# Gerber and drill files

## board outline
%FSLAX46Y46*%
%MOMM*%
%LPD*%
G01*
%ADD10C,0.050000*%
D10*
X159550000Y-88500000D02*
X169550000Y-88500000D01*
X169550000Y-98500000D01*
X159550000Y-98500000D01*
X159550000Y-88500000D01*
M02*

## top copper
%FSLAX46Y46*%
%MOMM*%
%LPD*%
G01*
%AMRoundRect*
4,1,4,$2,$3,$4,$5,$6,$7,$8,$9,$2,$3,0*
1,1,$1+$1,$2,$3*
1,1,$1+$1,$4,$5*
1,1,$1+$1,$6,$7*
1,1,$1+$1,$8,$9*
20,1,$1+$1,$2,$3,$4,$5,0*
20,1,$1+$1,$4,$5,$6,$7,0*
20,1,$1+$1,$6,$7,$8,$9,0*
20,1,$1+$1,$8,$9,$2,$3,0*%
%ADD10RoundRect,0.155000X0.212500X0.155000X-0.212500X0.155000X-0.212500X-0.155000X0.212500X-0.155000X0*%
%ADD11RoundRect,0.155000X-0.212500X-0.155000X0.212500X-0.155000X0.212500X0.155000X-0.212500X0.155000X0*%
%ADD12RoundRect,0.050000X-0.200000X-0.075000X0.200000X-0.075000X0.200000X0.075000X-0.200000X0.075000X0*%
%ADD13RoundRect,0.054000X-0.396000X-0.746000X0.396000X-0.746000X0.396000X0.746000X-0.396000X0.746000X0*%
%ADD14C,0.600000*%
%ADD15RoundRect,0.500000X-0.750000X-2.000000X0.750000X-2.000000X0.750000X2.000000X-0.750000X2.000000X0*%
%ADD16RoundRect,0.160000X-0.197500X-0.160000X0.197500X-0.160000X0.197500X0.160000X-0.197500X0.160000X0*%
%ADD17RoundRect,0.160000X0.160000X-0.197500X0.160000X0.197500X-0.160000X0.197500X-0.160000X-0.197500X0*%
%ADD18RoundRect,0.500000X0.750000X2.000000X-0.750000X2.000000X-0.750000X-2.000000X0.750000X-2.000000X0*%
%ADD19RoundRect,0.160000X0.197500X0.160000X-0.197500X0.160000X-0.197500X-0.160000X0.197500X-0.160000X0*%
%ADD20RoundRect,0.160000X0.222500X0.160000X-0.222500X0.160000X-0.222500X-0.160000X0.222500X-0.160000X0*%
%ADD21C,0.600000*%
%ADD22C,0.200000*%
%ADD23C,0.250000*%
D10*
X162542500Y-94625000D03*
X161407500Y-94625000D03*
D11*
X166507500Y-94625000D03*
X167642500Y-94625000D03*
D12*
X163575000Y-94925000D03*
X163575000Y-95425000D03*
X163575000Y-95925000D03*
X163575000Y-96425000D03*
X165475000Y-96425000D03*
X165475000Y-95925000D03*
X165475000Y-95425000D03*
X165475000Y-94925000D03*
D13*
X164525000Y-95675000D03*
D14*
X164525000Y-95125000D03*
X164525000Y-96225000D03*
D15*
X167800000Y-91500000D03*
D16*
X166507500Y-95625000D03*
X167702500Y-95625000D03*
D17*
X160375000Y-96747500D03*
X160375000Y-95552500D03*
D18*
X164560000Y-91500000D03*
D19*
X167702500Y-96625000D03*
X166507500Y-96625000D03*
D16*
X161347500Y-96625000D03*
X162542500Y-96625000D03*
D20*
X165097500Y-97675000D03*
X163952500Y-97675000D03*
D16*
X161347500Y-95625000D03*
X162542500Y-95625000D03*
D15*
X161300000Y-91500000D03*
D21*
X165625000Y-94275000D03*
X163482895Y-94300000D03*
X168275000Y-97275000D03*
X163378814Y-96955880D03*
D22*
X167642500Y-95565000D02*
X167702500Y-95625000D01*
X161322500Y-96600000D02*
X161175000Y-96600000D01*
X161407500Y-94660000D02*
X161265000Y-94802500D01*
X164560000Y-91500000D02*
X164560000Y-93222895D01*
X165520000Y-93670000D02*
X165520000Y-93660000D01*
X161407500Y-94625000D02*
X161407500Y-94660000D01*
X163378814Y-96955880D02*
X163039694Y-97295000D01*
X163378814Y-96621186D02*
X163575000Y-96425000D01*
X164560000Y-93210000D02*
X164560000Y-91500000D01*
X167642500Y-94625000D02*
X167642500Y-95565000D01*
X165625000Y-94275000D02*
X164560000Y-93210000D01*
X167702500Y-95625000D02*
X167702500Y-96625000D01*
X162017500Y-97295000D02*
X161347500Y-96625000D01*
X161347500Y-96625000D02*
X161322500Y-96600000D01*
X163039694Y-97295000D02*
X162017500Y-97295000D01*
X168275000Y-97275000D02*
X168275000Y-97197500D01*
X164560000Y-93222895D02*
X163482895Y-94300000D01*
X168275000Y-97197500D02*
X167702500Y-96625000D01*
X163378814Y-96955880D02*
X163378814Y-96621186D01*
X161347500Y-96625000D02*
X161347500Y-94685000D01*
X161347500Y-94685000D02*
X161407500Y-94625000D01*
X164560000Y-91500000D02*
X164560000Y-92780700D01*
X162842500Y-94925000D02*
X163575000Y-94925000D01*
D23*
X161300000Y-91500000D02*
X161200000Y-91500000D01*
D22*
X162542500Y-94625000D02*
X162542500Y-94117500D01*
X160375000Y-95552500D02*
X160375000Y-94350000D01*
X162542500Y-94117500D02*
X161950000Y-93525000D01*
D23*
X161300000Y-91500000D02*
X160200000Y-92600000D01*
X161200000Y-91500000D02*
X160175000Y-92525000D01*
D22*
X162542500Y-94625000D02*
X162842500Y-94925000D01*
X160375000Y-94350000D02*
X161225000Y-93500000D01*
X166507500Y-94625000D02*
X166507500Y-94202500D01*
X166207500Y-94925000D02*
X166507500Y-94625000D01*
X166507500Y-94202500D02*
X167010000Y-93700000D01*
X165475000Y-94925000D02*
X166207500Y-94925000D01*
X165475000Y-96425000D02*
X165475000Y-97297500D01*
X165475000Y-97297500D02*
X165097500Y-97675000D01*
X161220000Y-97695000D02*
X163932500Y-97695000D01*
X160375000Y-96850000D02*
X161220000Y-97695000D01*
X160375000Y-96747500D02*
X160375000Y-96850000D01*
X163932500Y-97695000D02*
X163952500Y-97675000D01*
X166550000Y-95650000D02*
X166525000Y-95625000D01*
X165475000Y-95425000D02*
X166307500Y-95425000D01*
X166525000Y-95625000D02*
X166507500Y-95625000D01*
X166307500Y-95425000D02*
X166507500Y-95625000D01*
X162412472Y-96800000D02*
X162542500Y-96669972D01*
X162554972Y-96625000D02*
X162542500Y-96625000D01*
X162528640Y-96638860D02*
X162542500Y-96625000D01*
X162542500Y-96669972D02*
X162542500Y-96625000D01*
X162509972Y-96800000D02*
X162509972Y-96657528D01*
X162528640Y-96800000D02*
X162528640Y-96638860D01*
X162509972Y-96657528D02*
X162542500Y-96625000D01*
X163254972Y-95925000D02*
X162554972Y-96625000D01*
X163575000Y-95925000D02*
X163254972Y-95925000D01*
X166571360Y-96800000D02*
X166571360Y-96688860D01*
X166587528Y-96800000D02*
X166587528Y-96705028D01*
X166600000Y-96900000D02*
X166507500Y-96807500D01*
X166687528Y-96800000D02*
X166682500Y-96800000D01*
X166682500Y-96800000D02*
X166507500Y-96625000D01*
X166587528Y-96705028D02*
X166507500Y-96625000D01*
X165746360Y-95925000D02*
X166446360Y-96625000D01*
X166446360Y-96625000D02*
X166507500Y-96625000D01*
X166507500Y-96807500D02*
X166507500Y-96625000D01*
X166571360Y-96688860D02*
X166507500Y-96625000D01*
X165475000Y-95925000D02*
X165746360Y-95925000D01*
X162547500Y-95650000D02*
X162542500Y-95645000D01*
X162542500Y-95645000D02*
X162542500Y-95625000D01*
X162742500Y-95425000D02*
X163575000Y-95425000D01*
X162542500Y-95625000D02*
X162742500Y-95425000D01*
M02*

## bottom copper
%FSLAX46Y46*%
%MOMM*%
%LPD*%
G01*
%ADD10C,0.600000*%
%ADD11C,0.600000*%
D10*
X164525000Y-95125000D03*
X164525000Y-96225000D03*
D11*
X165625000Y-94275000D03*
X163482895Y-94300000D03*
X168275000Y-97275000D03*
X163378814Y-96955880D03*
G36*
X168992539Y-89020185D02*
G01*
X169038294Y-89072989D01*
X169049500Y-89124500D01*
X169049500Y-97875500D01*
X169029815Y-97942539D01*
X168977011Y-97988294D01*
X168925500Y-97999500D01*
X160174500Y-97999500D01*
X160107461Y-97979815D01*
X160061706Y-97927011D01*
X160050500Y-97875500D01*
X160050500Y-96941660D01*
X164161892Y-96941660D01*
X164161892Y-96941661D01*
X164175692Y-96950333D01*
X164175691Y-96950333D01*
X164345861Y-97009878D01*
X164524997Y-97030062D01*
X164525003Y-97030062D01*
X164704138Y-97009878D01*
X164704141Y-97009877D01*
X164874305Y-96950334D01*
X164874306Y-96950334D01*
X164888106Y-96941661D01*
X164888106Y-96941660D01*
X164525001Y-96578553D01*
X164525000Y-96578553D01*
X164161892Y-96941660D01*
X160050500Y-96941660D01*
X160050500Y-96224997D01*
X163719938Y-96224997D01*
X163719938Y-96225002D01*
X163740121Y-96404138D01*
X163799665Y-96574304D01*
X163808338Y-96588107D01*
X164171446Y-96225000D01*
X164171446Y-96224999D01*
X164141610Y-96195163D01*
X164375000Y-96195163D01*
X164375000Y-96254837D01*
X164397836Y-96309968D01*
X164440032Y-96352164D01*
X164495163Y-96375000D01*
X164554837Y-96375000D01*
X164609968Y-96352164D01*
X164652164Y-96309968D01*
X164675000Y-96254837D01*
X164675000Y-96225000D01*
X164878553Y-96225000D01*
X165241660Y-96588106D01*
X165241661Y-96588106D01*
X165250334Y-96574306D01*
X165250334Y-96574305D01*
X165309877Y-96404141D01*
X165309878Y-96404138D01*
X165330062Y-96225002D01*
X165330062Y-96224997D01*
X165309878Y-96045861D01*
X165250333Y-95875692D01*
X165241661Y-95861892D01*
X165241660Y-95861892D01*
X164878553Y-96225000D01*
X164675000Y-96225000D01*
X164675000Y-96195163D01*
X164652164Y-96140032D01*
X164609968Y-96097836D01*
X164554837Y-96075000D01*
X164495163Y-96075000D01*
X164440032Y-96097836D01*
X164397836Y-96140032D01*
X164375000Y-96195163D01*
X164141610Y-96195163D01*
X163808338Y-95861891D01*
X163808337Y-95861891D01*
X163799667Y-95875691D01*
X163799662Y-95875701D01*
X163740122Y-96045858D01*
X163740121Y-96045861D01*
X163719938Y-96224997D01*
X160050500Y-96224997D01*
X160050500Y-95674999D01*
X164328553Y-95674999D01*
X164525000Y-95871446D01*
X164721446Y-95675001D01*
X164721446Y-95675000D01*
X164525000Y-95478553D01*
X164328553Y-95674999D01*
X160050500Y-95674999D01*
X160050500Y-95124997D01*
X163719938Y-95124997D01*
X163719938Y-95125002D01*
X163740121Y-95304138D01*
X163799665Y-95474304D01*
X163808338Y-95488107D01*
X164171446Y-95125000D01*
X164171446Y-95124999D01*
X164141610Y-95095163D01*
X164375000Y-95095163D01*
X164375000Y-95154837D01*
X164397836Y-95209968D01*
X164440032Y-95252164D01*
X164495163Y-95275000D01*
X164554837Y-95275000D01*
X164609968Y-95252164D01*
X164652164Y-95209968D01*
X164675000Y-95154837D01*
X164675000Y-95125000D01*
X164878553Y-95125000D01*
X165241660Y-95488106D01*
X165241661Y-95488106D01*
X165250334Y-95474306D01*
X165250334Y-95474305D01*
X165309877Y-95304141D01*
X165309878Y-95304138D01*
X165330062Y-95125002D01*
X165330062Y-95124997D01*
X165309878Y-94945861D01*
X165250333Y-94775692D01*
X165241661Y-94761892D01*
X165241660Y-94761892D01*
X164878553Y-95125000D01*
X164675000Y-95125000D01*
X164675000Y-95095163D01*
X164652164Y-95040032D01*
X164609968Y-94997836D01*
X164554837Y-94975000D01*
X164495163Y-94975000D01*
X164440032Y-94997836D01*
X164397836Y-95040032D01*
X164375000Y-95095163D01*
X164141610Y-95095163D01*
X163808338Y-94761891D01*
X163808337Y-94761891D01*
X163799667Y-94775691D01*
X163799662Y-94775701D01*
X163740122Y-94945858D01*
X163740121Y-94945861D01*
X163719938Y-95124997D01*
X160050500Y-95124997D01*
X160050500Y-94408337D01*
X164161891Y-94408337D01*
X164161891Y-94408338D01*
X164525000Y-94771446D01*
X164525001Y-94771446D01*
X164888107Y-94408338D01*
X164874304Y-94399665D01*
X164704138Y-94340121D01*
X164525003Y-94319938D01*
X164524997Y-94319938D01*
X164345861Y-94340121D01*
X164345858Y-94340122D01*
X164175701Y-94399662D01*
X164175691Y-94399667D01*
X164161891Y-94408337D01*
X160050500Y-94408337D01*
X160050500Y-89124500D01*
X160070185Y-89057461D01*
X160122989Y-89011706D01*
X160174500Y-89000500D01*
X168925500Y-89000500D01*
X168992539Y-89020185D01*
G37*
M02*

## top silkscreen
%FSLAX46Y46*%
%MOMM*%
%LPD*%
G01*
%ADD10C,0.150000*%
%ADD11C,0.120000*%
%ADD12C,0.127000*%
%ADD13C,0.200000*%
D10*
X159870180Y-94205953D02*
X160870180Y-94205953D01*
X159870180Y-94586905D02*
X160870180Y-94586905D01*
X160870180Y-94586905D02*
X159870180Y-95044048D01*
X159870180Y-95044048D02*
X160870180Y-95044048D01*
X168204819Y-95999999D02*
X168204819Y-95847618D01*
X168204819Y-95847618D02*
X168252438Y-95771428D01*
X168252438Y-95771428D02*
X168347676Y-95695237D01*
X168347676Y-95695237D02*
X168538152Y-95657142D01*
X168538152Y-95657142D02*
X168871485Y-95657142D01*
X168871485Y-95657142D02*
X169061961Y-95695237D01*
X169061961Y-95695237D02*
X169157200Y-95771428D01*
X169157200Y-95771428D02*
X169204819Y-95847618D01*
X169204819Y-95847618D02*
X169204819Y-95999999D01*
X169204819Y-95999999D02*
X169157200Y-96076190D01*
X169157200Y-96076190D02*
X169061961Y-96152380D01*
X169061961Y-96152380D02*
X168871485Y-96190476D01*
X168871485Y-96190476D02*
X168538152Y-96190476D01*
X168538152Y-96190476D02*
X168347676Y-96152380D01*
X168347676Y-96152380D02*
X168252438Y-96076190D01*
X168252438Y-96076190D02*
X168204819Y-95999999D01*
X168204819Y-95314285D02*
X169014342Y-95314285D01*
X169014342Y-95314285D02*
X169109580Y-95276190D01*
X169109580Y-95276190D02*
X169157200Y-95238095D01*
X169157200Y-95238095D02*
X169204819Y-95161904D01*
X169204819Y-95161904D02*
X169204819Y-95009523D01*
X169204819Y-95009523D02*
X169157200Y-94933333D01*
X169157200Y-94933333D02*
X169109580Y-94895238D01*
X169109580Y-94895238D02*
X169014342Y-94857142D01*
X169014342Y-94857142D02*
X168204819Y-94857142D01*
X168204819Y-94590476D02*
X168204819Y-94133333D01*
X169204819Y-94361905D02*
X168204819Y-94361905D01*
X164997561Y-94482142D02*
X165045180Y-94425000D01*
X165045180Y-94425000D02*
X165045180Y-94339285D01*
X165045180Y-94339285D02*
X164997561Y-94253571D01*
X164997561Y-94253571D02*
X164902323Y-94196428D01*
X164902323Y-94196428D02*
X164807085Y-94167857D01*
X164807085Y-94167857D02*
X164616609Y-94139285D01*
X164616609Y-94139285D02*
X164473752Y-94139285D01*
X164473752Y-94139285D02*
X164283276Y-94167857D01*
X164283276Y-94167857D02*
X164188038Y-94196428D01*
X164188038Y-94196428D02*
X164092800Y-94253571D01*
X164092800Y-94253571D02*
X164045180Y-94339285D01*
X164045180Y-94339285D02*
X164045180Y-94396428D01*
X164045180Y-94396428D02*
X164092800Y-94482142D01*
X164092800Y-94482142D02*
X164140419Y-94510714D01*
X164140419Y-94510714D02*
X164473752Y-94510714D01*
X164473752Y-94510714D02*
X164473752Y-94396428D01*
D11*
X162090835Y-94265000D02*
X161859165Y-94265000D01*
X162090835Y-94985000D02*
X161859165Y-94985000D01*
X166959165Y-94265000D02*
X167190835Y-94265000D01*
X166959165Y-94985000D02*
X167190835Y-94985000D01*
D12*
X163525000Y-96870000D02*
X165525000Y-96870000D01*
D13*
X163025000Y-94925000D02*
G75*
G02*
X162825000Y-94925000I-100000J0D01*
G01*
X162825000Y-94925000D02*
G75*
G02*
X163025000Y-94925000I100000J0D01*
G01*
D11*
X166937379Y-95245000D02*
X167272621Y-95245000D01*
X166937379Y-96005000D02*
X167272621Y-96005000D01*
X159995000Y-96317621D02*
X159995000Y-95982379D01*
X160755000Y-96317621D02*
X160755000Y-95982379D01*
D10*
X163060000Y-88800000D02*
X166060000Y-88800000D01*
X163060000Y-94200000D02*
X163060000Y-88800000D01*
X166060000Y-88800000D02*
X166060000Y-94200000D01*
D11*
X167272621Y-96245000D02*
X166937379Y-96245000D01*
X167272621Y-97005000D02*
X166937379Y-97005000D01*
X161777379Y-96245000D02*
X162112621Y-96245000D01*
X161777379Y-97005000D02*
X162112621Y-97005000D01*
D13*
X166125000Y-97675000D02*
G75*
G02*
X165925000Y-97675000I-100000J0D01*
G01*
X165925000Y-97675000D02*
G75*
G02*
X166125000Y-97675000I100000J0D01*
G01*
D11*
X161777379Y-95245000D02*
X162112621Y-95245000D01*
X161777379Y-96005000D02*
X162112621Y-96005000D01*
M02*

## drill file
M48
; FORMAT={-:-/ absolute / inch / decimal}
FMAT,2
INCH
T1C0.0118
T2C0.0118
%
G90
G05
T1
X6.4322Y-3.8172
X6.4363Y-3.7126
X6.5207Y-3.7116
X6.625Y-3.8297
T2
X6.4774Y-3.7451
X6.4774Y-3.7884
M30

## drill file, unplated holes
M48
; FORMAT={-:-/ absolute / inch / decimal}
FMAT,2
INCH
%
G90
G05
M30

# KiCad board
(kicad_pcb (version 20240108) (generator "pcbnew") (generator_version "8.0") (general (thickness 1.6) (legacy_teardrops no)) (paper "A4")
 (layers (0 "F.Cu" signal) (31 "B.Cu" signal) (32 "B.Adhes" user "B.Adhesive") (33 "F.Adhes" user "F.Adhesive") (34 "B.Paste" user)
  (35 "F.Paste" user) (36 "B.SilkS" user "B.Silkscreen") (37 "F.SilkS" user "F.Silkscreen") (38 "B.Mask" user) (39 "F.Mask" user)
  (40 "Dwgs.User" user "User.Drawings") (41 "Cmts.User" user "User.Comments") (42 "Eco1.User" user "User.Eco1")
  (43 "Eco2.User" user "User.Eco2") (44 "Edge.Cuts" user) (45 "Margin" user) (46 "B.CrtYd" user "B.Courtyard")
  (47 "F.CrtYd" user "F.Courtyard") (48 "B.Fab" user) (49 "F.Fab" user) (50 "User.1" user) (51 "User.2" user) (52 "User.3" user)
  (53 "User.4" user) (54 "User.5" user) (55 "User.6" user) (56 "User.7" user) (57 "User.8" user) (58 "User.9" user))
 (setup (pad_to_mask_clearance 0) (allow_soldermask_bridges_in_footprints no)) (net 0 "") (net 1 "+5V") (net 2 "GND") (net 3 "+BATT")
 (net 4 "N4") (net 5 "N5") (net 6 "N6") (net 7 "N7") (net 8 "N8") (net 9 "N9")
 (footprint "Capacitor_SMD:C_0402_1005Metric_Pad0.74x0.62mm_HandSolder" (layer "F.Cu") (at 161.975 94.625 180)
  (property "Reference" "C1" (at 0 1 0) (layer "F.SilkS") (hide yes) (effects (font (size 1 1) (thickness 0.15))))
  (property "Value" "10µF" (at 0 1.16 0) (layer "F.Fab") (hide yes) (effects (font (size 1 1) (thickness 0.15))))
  (fp_line (start -0.115835 0.36) (end 0.115835 0.36) (stroke (width 0.12) (type solid)) (layer "F.SilkS"))
  (fp_line (start -0.115835 -0.36) (end 0.115835 -0.36) (stroke (width 0.12) (type solid)) (layer "F.SilkS"))
  (pad "1" smd roundrect (at -0.5675 0 180) (size 0.735 0.62) (layers "F.Cu" "F.Paste" "F.Mask") (roundrect_rratio 0.25) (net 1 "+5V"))
  (pad "2" smd roundrect (at 0.5675 0 180) (size 0.735 0.62) (layers "F.Cu" "F.Paste" "F.Mask") (roundrect_rratio 0.25) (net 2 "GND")))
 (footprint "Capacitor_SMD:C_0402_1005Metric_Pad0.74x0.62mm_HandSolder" (layer "F.Cu") (at 167.075 94.625)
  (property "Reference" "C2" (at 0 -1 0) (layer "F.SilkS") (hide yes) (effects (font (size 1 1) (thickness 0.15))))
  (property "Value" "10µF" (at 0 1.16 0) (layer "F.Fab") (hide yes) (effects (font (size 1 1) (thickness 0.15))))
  (fp_line (start -0.115835 -0.36) (end 0.115835 -0.36) (stroke (width 0.12) (type solid)) (layer "F.SilkS"))
  (fp_line (start -0.115835 0.36) (end 0.115835 0.36) (stroke (width 0.12) (type solid)) (layer "F.SilkS"))
  (pad "1" smd roundrect (at -0.5675 0) (size 0.735 0.62) (layers "F.Cu" "F.Paste" "F.Mask") (roundrect_rratio 0.25) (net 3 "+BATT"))
  (pad "2" smd roundrect (at 0.5675 0) (size 0.735 0.62) (layers "F.Cu" "F.Paste" "F.Mask") (roundrect_rratio 0.25) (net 2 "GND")))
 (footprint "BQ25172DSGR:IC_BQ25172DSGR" (layer "F.Cu") (at 164.525 95.675)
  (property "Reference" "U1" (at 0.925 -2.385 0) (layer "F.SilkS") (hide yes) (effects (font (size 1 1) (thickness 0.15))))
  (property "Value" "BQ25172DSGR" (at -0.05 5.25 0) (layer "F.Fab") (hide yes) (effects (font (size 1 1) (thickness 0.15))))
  (fp_line (start -1 1.195) (end 1 1.195) (stroke (width 0.127) (type solid)) (layer "F.SilkS"))
  (fp_circle (center -1.6 -0.75) (end -1.5 -0.75) (stroke (width 0.2) (type solid)) (fill none) (layer "F.SilkS"))
  (pad "1" smd roundrect (at -0.95 -0.75) (size 0.5 0.25) (layers "F.Cu" "F.Paste" "F.Mask") (roundrect_rratio 0.2) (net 1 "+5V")
   (solder_mask_margin 0.102))
  (pad "2" smd roundrect (at -0.95 -0.25) (size 0.5 0.25) (layers "F.Cu" "F.Paste" "F.Mask") (roundrect_rratio 0.2) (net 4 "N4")
   (solder_mask_margin 0.102))
  (pad "3" smd roundrect (at -0.95 0.25) (size 0.5 0.25) (layers "F.Cu" "F.Paste" "F.Mask") (roundrect_rratio 0.2) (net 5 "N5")
   (solder_mask_margin 0.102))
  (pad "4" smd roundrect (at -0.95 0.75) (size 0.5 0.25) (layers "F.Cu" "F.Paste" "F.Mask") (roundrect_rratio 0.2) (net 2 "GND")
   (solder_mask_margin 0.102))
  (pad "5" smd roundrect (at 0.95 0.75) (size 0.5 0.25) (layers "F.Cu" "F.Paste" "F.Mask") (roundrect_rratio 0.2) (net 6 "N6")
   (solder_mask_margin 0.102))
  (pad "6" smd roundrect (at 0.95 0.25) (size 0.5 0.25) (layers "F.Cu" "F.Paste" "F.Mask") (roundrect_rratio 0.2) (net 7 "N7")
   (solder_mask_margin 0.102))
  (pad "7" smd roundrect (at 0.95 -0.25) (size 0.5 0.25) (layers "F.Cu" "F.Paste" "F.Mask") (roundrect_rratio 0.2) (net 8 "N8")
   (solder_mask_margin 0.102))
  (pad "8" smd roundrect (at 0.95 -0.75) (size 0.5 0.25) (layers "F.Cu" "F.Paste" "F.Mask") (roundrect_rratio 0.2) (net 3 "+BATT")
   (solder_mask_margin 0.102))
  (pad "9" smd roundrect (at 0 0) (size 0.9 1.6) (layers "F.Cu" "F.Mask") (roundrect_rratio 0.06) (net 2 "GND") (solder_mask_margin 0.102))
  (pad "10" thru_hole circle (at 0 -0.55) (size 0.6 0.6) (drill 0.3) (layers "*.Cu") (remove_unused_layers no) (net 2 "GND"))
  (pad "11" thru_hole circle (at 0 0.55) (size 0.6 0.6) (drill 0.3) (layers "*.Cu") (remove_unused_layers no) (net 2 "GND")))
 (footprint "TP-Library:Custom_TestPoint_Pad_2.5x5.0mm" (layer "F.Cu") (at 167.8 90)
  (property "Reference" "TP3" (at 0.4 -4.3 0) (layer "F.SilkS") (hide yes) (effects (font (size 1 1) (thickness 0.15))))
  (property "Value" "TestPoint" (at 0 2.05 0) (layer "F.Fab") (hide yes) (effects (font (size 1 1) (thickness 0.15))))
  (pad "1" smd roundrect (at 0 1.5) (size 2.5 5) (layers "F.Cu" "F.Mask") (roundrect_rratio 0.2) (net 3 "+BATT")))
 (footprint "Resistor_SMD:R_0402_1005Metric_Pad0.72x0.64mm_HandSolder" (layer "F.Cu") (at 167.105 95.625)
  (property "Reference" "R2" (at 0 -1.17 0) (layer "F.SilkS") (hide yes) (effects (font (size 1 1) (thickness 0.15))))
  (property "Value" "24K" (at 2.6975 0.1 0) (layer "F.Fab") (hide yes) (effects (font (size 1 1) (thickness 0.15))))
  (fp_line (start -0.167621 -0.38) (end 0.167621 -0.38) (stroke (width 0.12) (type solid)) (layer "F.SilkS"))
  (fp_line (start -0.167621 0.38) (end 0.167621 0.38) (stroke (width 0.12) (type solid)) (layer "F.SilkS"))
  (pad "1" smd roundrect (at -0.5975 0) (size 0.715 0.64) (layers "F.Cu" "F.Paste" "F.Mask") (roundrect_rratio 0.25) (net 8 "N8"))
  (pad "2" smd roundrect (at 0.5975 0) (size 0.715 0.64) (layers "F.Cu" "F.Paste" "F.Mask") (roundrect_rratio 0.25) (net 2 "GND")))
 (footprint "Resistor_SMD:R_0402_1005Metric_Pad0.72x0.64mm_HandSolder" (layer "F.Cu") (at 160.375 96.15 90)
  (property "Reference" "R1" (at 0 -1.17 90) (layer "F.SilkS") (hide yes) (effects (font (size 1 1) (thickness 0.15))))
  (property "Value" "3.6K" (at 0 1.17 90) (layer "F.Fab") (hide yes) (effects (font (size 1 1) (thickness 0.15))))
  (fp_line (start -0.167621 -0.38) (end 0.167621 -0.38) (stroke (width 0.12) (type solid)) (layer "F.SilkS"))
  (fp_line (start -0.167621 0.38) (end 0.167621 0.38) (stroke (width 0.12) (type solid)) (layer "F.SilkS"))
  (pad "1" smd roundrect (at -0.5975 0 90) (size 0.715 0.64) (layers "F.Cu" "F.Paste" "F.Mask") (roundrect_rratio 0.25) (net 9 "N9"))
  (pad "2" smd roundrect (at 0.5975 0 90) (size 0.715 0.64) (layers "F.Cu" "F.Paste" "F.Mask") (roundrect_rratio 0.25) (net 1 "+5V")))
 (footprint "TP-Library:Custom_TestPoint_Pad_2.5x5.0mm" (layer "F.Cu") (at 164.56 93 180)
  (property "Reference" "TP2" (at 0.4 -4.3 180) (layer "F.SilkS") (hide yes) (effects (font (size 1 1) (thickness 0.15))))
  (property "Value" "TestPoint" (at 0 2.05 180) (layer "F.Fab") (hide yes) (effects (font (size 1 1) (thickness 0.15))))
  (fp_line (start 1.5 4.2) (end -1.5 4.2) (stroke (width 0.15) (type default)) (layer "F.SilkS"))
  (fp_line (start 1.5 -1.2) (end 1.5 4.2) (stroke (width 0.15) (type default)) (layer "F.SilkS"))
  (fp_line (start -1.5 4.2) (end -1.5 -1.2) (stroke (width 0.15) (type default)) (layer "F.SilkS"))
  (pad "1" smd roundrect (at 0 1.5 180) (size 2.5 5) (layers "F.Cu" "F.Mask") (roundrect_rratio 0.2) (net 2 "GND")))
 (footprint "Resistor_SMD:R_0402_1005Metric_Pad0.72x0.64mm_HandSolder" (layer "F.Cu") (at 167.105 96.625 180)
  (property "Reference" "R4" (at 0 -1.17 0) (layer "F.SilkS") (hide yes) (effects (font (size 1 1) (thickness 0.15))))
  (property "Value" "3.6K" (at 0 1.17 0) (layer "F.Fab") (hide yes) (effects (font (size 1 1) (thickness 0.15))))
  (fp_line (start -0.167621 0.38) (end 0.167621 0.38) (stroke (width 0.12) (type solid)) (layer "F.SilkS"))
  (fp_line (start -0.167621 -0.38) (end 0.167621 -0.38) (stroke (width 0.12) (type solid)) (layer "F.SilkS"))
  (pad "1" smd roundrect (at -0.5975 0 180) (size 0.715 0.64) (layers "F.Cu" "F.Paste" "F.Mask") (roundrect_rratio 0.25) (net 2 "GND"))
  (pad "2" smd roundrect (at 0.5975 0 180) (size 0.715 0.64) (layers "F.Cu" "F.Paste" "F.Mask") (roundrect_rratio 0.25) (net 7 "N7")))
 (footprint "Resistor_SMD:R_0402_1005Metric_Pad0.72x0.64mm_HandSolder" (layer "F.Cu") (at 161.945 96.625)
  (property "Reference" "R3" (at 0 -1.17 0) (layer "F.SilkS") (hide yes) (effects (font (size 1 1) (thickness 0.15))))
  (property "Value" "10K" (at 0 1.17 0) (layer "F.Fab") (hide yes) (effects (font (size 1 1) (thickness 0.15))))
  (fp_line (start -0.167621 -0.38) (end 0.167621 -0.38) (stroke (width 0.12) (type solid)) (layer "F.SilkS"))
  (fp_line (start -0.167621 0.38) (end 0.167621 0.38) (stroke (width 0.12) (type solid)) (layer "F.SilkS"))
  (pad "1" smd roundrect (at -0.5975 0) (size 0.715 0.64) (layers "F.Cu" "F.Paste" "F.Mask") (roundrect_rratio 0.25) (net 2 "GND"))
  (pad "2" smd roundrect (at 0.5975 0) (size 0.715 0.64) (layers "F.Cu" "F.Paste" "F.Mask") (roundrect_rratio 0.25) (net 5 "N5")))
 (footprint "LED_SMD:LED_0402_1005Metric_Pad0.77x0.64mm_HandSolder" (layer "F.Cu") (at 164.525 97.675 180)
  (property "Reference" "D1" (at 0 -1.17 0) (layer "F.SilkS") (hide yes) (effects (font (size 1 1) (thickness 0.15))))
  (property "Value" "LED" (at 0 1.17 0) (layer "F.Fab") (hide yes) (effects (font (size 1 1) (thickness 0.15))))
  (fp_circle (center -1.5 0) (end -1.4 0) (stroke (width 0.2) (type solid)) (fill solid) (layer "F.SilkS"))
  (pad "1" smd roundrect (at -0.5725 0 180) (size 0.765 0.64) (layers "F.Cu" "F.Paste" "F.Mask") (roundrect_rratio 0.25) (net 6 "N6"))
  (pad "2" smd roundrect (at 0.5725 0 180) (size 0.765 0.64) (layers "F.Cu" "F.Paste" "F.Mask") (roundrect_rratio 0.25) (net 9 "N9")))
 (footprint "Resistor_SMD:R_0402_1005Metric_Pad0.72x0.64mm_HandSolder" (layer "F.Cu") (at 161.945 95.625)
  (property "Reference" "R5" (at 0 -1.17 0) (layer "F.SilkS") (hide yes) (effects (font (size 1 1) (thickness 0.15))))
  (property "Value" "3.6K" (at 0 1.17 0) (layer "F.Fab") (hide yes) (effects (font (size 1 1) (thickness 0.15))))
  (fp_line (start -0.167621 -0.38) (end 0.167621 -0.38) (stroke (width 0.12) (type solid)) (layer "F.SilkS"))
  (fp_line (start -0.167621 0.38) (end 0.167621 0.38) (stroke (width 0.12) (type solid)) (layer "F.SilkS"))
  (pad "1" smd roundrect (at -0.5975 0) (size 0.715 0.64) (layers "F.Cu" "F.Paste" "F.Mask") (roundrect_rratio 0.25) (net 2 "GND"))
  (pad "2" smd roundrect (at 0.5975 0) (size 0.715 0.64) (layers "F.Cu" "F.Paste" "F.Mask") (roundrect_rratio 0.25) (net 4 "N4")))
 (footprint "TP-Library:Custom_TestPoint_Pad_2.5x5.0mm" (layer "F.Cu") (at 161.3 90)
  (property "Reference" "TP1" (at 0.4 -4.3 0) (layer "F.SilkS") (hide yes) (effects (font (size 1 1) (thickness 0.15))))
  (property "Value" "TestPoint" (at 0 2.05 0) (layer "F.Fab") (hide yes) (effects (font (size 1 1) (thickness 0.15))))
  (pad "1" smd roundrect (at 0 1.5) (size 2.5 5) (layers "F.Cu" "F.Mask") (roundrect_rratio 0.2) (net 1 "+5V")))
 (gr_rect (start 159.55 88.5) (end 169.55 98.5) (stroke (width 0.05) (type default)) (fill none) (layer "Edge.Cuts"))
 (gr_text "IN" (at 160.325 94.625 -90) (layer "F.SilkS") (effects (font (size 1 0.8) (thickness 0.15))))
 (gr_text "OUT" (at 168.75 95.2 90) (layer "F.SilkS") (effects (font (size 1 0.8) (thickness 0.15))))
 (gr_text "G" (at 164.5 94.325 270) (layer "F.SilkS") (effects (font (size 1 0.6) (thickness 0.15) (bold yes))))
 (segment (start 167.6425 95.565) (end 167.7025 95.625) (width 0.2) (layer "F.Cu") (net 2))
 (segment (start 161.3225 96.6) (end 161.175 96.6) (width 0.2) (layer "F.Cu") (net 2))
 (segment (start 161.4075 94.66) (end 161.265 94.8025) (width 0.2) (layer "F.Cu") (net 2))
 (segment (start 164.56 91.5) (end 164.56 93.222895) (width 0.2) (layer "F.Cu") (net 2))
 (segment (start 165.52 93.67) (end 165.52 93.66) (width 0.2) (layer "F.Cu") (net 2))
 (segment (start 161.4075 94.625) (end 161.4075 94.66) (width 0.2) (layer "F.Cu") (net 2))
 (segment (start 163.378814 96.95588) (end 163.039694 97.295) (width 0.2) (layer "F.Cu") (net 2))
 (segment (start 163.378814 96.621186) (end 163.575 96.425) (width 0.2) (layer "F.Cu") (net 2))
 (segment (start 164.56 93.21) (end 164.56 91.5) (width 0.2) (layer "F.Cu") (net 2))
 (segment (start 167.6425 94.625) (end 167.6425 95.565) (width 0.2) (layer "F.Cu") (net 2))
 (segment (start 165.625 94.275) (end 164.56 93.21) (width 0.2) (layer "F.Cu") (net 2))
 (segment (start 167.7025 95.625) (end 167.7025 96.625) (width 0.2) (layer "F.Cu") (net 2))
 (segment (start 162.0175 97.295) (end 161.3475 96.625) (width 0.2) (layer "F.Cu") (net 2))
 (segment (start 161.3475 96.625) (end 161.3225 96.6) (width 0.2) (layer "F.Cu") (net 2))
 (segment (start 163.039694 97.295) (end 162.0175 97.295) (width 0.2) (layer "F.Cu") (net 2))
 (segment (start 168.275 97.275) (end 168.275 97.1975) (width 0.2) (layer "F.Cu") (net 2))
 (segment (start 164.56 93.222895) (end 163.482895 94.3) (width 0.2) (layer "F.Cu") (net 2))
 (segment (start 168.275 97.1975) (end 167.7025 96.625) (width 0.2) (layer "F.Cu") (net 2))
 (segment (start 163.378814 96.95588) (end 163.378814 96.621186) (width 0.2) (layer "F.Cu") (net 2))
 (segment (start 161.3475 96.625) (end 161.3475 94.685) (width 0.2) (layer "F.Cu") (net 2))
 (segment (start 161.3475 94.685) (end 161.4075 94.625) (width 0.2) (layer "F.Cu") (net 2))
 (segment (start 164.56 91.5) (end 164.56 92.7807) (width 0.2) (layer "F.Cu") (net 2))
 (via (at 165.625 94.275) (size 0.6) (drill 0.3) (layers "F.Cu" "B.Cu") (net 2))
 (via (at 163.482895 94.3) (size 0.6) (drill 0.3) (layers "F.Cu" "B.Cu") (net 2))
 (via (at 168.275 97.275) (size 0.6) (drill 0.3) (layers "F.Cu" "B.Cu") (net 2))
 (via (at 163.378814 96.95588) (size 0.6) (drill 0.3) (layers "F.Cu" "B.Cu") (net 2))
 (segment (start 162.8425 94.925) (end 163.575 94.925) (width 0.2) (layer "F.Cu") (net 1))
 (segment (start 161.3 91.5) (end 161.2 91.5) (width 0.25) (layer "F.Cu") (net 1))
 (segment (start 162.5425 94.625) (end 162.5425 94.1175) (width 0.2) (layer "F.Cu") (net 1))
 (segment (start 160.375 95.5525) (end 160.375 94.35) (width 0.2) (layer "F.Cu") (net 1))
 (segment (start 162.5425 94.1175) (end 161.95 93.525) (width 0.2) (layer "F.Cu") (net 1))
 (segment (start 161.3 91.5) (end 160.2 92.6) (width 0.25) (layer "F.Cu") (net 1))
 (segment (start 161.2 91.5) (end 160.175 92.525) (width 0.25) (layer "F.Cu") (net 1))
 (segment (start 162.5425 94.625) (end 162.8425 94.925) (width 0.2) (layer "F.Cu") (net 1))
 (segment (start 160.375 94.35) (end 161.225 93.5) (width 0.2) (layer "F.Cu") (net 1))
 (segment (start 166.5075 94.625) (end 166.5075 94.2025) (width 0.2) (layer "F.Cu") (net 3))
 (segment (start 166.2075 94.925) (end 166.5075 94.625) (width 0.2) (layer "F.Cu") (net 3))
 (segment (start 166.5075 94.2025) (end 167.01 93.7) (width 0.2) (layer "F.Cu") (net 3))
 (segment (start 165.475 94.925) (end 166.2075 94.925) (width 0.2) (layer "F.Cu") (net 3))
 (segment (start 165.475 96.425) (end 165.475 97.2975) (width 0.2) (layer "F.Cu") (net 6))
 (segment (start 165.475 97.2975) (end 165.0975 97.675) (width 0.2) (layer "F.Cu") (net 6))
 (segment (start 161.22 97.695) (end 163.9325 97.695) (width 0.2) (layer "F.Cu") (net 9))
 (segment (start 160.375 96.85) (end 161.22 97.695) (width 0.2) (layer "F.Cu") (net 9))
 (segment (start 160.375 96.7475) (end 160.375 96.85) (width 0.2) (layer "F.Cu") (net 9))
 (segment (start 163.9325 97.695) (end 163.9525 97.675) (width 0.2) (layer "F.Cu") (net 9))
 (segment (start 166.55 95.65) (end 166.525 95.625) (width 0.2) (layer "F.Cu") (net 8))
 (segment (start 165.475 95.425) (end 166.3075 95.425) (width 0.2) (layer "F.Cu") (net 8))
 (segment (start 166.525 95.625) (end 166.5075 95.625) (width 0.2) (layer "F.Cu") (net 8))
 (segment (start 166.3075 95.425) (end 166.5075 95.625) (width 0.2) (layer "F.Cu") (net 8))
 (segment (start 162.412472 96.8) (end 162.5425 96.669972) (width 0.2) (layer "F.Cu") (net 5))
 (segment (start 162.554972 96.625) (end 162.5425 96.625) (width 0.2) (layer "F.Cu") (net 5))
 (segment (start 162.52864 96.63886) (end 162.5425 96.625) (width 0.2) (layer "F.Cu") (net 5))
 (segment (start 162.5425 96.669972) (end 162.5425 96.625) (width 0.2) (layer "F.Cu") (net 5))
 (segment (start 162.509972 96.8) (end 162.509972 96.657528) (width 0.2) (layer "F.Cu") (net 5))
 (segment (start 162.52864 96.8) (end 162.52864 96.63886) (width 0.2) (layer "F.Cu") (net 5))
 (segment (start 162.509972 96.657528) (end 162.5425 96.625) (width 0.2) (layer "F.Cu") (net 5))
 (segment (start 163.254972 95.925) (end 162.554972 96.625) (width 0.2) (layer "F.Cu") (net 5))
 (segment (start 163.575 95.925) (end 163.254972 95.925) (width 0.2) (layer "F.Cu") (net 5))
 (segment (start 166.57136 96.8) (end 166.57136 96.68886) (width 0.2) (layer "F.Cu") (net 7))
 (segment (start 166.587528 96.8) (end 166.587528 96.705028) (width 0.2) (layer "F.Cu") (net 7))
 (segment (start 166.6 96.9) (end 166.5075 96.8075) (width 0.2) (layer "F.Cu") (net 7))
 (segment (start 166.687528 96.8) (end 166.6825 96.8) (width 0.2) (layer "F.Cu") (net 7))
 (segment (start 166.6825 96.8) (end 166.5075 96.625) (width 0.2) (layer "F.Cu") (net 7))
 (segment (start 166.587528 96.705028) (end 166.5075 96.625) (width 0.2) (layer "F.Cu") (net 7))
 (segment (start 165.74636 95.925) (end 166.44636 96.625) (width 0.2) (layer "F.Cu") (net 7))
 (segment (start 166.44636 96.625) (end 166.5075 96.625) (width 0.2) (layer "F.Cu") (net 7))
 (segment (start 166.5075 96.8075) (end 166.5075 96.625) (width 0.2) (layer "F.Cu") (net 7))
 (segment (start 166.57136 96.68886) (end 166.5075 96.625) (width 0.2) (layer "F.Cu") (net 7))
 (segment (start 165.475 95.925) (end 165.74636 95.925) (width 0.2) (layer "F.Cu") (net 7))
 (segment (start 162.5475 95.65) (end 162.5425 95.645) (width 0.2) (layer "F.Cu") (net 4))
 (segment (start 162.5425 95.645) (end 162.5425 95.625) (width 0.2) (layer "F.Cu") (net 4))
 (segment (start 162.7425 95.425) (end 163.575 95.425) (width 0.2) (layer "F.Cu") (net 4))
 (segment (start 162.5425 95.625) (end 162.7425 95.425) (width 0.2) (layer "F.Cu") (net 4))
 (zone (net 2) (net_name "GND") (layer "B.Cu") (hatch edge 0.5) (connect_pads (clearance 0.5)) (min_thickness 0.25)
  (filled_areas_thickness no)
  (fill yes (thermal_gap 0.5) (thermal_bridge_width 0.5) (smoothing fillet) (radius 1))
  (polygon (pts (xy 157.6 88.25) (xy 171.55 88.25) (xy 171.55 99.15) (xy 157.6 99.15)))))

